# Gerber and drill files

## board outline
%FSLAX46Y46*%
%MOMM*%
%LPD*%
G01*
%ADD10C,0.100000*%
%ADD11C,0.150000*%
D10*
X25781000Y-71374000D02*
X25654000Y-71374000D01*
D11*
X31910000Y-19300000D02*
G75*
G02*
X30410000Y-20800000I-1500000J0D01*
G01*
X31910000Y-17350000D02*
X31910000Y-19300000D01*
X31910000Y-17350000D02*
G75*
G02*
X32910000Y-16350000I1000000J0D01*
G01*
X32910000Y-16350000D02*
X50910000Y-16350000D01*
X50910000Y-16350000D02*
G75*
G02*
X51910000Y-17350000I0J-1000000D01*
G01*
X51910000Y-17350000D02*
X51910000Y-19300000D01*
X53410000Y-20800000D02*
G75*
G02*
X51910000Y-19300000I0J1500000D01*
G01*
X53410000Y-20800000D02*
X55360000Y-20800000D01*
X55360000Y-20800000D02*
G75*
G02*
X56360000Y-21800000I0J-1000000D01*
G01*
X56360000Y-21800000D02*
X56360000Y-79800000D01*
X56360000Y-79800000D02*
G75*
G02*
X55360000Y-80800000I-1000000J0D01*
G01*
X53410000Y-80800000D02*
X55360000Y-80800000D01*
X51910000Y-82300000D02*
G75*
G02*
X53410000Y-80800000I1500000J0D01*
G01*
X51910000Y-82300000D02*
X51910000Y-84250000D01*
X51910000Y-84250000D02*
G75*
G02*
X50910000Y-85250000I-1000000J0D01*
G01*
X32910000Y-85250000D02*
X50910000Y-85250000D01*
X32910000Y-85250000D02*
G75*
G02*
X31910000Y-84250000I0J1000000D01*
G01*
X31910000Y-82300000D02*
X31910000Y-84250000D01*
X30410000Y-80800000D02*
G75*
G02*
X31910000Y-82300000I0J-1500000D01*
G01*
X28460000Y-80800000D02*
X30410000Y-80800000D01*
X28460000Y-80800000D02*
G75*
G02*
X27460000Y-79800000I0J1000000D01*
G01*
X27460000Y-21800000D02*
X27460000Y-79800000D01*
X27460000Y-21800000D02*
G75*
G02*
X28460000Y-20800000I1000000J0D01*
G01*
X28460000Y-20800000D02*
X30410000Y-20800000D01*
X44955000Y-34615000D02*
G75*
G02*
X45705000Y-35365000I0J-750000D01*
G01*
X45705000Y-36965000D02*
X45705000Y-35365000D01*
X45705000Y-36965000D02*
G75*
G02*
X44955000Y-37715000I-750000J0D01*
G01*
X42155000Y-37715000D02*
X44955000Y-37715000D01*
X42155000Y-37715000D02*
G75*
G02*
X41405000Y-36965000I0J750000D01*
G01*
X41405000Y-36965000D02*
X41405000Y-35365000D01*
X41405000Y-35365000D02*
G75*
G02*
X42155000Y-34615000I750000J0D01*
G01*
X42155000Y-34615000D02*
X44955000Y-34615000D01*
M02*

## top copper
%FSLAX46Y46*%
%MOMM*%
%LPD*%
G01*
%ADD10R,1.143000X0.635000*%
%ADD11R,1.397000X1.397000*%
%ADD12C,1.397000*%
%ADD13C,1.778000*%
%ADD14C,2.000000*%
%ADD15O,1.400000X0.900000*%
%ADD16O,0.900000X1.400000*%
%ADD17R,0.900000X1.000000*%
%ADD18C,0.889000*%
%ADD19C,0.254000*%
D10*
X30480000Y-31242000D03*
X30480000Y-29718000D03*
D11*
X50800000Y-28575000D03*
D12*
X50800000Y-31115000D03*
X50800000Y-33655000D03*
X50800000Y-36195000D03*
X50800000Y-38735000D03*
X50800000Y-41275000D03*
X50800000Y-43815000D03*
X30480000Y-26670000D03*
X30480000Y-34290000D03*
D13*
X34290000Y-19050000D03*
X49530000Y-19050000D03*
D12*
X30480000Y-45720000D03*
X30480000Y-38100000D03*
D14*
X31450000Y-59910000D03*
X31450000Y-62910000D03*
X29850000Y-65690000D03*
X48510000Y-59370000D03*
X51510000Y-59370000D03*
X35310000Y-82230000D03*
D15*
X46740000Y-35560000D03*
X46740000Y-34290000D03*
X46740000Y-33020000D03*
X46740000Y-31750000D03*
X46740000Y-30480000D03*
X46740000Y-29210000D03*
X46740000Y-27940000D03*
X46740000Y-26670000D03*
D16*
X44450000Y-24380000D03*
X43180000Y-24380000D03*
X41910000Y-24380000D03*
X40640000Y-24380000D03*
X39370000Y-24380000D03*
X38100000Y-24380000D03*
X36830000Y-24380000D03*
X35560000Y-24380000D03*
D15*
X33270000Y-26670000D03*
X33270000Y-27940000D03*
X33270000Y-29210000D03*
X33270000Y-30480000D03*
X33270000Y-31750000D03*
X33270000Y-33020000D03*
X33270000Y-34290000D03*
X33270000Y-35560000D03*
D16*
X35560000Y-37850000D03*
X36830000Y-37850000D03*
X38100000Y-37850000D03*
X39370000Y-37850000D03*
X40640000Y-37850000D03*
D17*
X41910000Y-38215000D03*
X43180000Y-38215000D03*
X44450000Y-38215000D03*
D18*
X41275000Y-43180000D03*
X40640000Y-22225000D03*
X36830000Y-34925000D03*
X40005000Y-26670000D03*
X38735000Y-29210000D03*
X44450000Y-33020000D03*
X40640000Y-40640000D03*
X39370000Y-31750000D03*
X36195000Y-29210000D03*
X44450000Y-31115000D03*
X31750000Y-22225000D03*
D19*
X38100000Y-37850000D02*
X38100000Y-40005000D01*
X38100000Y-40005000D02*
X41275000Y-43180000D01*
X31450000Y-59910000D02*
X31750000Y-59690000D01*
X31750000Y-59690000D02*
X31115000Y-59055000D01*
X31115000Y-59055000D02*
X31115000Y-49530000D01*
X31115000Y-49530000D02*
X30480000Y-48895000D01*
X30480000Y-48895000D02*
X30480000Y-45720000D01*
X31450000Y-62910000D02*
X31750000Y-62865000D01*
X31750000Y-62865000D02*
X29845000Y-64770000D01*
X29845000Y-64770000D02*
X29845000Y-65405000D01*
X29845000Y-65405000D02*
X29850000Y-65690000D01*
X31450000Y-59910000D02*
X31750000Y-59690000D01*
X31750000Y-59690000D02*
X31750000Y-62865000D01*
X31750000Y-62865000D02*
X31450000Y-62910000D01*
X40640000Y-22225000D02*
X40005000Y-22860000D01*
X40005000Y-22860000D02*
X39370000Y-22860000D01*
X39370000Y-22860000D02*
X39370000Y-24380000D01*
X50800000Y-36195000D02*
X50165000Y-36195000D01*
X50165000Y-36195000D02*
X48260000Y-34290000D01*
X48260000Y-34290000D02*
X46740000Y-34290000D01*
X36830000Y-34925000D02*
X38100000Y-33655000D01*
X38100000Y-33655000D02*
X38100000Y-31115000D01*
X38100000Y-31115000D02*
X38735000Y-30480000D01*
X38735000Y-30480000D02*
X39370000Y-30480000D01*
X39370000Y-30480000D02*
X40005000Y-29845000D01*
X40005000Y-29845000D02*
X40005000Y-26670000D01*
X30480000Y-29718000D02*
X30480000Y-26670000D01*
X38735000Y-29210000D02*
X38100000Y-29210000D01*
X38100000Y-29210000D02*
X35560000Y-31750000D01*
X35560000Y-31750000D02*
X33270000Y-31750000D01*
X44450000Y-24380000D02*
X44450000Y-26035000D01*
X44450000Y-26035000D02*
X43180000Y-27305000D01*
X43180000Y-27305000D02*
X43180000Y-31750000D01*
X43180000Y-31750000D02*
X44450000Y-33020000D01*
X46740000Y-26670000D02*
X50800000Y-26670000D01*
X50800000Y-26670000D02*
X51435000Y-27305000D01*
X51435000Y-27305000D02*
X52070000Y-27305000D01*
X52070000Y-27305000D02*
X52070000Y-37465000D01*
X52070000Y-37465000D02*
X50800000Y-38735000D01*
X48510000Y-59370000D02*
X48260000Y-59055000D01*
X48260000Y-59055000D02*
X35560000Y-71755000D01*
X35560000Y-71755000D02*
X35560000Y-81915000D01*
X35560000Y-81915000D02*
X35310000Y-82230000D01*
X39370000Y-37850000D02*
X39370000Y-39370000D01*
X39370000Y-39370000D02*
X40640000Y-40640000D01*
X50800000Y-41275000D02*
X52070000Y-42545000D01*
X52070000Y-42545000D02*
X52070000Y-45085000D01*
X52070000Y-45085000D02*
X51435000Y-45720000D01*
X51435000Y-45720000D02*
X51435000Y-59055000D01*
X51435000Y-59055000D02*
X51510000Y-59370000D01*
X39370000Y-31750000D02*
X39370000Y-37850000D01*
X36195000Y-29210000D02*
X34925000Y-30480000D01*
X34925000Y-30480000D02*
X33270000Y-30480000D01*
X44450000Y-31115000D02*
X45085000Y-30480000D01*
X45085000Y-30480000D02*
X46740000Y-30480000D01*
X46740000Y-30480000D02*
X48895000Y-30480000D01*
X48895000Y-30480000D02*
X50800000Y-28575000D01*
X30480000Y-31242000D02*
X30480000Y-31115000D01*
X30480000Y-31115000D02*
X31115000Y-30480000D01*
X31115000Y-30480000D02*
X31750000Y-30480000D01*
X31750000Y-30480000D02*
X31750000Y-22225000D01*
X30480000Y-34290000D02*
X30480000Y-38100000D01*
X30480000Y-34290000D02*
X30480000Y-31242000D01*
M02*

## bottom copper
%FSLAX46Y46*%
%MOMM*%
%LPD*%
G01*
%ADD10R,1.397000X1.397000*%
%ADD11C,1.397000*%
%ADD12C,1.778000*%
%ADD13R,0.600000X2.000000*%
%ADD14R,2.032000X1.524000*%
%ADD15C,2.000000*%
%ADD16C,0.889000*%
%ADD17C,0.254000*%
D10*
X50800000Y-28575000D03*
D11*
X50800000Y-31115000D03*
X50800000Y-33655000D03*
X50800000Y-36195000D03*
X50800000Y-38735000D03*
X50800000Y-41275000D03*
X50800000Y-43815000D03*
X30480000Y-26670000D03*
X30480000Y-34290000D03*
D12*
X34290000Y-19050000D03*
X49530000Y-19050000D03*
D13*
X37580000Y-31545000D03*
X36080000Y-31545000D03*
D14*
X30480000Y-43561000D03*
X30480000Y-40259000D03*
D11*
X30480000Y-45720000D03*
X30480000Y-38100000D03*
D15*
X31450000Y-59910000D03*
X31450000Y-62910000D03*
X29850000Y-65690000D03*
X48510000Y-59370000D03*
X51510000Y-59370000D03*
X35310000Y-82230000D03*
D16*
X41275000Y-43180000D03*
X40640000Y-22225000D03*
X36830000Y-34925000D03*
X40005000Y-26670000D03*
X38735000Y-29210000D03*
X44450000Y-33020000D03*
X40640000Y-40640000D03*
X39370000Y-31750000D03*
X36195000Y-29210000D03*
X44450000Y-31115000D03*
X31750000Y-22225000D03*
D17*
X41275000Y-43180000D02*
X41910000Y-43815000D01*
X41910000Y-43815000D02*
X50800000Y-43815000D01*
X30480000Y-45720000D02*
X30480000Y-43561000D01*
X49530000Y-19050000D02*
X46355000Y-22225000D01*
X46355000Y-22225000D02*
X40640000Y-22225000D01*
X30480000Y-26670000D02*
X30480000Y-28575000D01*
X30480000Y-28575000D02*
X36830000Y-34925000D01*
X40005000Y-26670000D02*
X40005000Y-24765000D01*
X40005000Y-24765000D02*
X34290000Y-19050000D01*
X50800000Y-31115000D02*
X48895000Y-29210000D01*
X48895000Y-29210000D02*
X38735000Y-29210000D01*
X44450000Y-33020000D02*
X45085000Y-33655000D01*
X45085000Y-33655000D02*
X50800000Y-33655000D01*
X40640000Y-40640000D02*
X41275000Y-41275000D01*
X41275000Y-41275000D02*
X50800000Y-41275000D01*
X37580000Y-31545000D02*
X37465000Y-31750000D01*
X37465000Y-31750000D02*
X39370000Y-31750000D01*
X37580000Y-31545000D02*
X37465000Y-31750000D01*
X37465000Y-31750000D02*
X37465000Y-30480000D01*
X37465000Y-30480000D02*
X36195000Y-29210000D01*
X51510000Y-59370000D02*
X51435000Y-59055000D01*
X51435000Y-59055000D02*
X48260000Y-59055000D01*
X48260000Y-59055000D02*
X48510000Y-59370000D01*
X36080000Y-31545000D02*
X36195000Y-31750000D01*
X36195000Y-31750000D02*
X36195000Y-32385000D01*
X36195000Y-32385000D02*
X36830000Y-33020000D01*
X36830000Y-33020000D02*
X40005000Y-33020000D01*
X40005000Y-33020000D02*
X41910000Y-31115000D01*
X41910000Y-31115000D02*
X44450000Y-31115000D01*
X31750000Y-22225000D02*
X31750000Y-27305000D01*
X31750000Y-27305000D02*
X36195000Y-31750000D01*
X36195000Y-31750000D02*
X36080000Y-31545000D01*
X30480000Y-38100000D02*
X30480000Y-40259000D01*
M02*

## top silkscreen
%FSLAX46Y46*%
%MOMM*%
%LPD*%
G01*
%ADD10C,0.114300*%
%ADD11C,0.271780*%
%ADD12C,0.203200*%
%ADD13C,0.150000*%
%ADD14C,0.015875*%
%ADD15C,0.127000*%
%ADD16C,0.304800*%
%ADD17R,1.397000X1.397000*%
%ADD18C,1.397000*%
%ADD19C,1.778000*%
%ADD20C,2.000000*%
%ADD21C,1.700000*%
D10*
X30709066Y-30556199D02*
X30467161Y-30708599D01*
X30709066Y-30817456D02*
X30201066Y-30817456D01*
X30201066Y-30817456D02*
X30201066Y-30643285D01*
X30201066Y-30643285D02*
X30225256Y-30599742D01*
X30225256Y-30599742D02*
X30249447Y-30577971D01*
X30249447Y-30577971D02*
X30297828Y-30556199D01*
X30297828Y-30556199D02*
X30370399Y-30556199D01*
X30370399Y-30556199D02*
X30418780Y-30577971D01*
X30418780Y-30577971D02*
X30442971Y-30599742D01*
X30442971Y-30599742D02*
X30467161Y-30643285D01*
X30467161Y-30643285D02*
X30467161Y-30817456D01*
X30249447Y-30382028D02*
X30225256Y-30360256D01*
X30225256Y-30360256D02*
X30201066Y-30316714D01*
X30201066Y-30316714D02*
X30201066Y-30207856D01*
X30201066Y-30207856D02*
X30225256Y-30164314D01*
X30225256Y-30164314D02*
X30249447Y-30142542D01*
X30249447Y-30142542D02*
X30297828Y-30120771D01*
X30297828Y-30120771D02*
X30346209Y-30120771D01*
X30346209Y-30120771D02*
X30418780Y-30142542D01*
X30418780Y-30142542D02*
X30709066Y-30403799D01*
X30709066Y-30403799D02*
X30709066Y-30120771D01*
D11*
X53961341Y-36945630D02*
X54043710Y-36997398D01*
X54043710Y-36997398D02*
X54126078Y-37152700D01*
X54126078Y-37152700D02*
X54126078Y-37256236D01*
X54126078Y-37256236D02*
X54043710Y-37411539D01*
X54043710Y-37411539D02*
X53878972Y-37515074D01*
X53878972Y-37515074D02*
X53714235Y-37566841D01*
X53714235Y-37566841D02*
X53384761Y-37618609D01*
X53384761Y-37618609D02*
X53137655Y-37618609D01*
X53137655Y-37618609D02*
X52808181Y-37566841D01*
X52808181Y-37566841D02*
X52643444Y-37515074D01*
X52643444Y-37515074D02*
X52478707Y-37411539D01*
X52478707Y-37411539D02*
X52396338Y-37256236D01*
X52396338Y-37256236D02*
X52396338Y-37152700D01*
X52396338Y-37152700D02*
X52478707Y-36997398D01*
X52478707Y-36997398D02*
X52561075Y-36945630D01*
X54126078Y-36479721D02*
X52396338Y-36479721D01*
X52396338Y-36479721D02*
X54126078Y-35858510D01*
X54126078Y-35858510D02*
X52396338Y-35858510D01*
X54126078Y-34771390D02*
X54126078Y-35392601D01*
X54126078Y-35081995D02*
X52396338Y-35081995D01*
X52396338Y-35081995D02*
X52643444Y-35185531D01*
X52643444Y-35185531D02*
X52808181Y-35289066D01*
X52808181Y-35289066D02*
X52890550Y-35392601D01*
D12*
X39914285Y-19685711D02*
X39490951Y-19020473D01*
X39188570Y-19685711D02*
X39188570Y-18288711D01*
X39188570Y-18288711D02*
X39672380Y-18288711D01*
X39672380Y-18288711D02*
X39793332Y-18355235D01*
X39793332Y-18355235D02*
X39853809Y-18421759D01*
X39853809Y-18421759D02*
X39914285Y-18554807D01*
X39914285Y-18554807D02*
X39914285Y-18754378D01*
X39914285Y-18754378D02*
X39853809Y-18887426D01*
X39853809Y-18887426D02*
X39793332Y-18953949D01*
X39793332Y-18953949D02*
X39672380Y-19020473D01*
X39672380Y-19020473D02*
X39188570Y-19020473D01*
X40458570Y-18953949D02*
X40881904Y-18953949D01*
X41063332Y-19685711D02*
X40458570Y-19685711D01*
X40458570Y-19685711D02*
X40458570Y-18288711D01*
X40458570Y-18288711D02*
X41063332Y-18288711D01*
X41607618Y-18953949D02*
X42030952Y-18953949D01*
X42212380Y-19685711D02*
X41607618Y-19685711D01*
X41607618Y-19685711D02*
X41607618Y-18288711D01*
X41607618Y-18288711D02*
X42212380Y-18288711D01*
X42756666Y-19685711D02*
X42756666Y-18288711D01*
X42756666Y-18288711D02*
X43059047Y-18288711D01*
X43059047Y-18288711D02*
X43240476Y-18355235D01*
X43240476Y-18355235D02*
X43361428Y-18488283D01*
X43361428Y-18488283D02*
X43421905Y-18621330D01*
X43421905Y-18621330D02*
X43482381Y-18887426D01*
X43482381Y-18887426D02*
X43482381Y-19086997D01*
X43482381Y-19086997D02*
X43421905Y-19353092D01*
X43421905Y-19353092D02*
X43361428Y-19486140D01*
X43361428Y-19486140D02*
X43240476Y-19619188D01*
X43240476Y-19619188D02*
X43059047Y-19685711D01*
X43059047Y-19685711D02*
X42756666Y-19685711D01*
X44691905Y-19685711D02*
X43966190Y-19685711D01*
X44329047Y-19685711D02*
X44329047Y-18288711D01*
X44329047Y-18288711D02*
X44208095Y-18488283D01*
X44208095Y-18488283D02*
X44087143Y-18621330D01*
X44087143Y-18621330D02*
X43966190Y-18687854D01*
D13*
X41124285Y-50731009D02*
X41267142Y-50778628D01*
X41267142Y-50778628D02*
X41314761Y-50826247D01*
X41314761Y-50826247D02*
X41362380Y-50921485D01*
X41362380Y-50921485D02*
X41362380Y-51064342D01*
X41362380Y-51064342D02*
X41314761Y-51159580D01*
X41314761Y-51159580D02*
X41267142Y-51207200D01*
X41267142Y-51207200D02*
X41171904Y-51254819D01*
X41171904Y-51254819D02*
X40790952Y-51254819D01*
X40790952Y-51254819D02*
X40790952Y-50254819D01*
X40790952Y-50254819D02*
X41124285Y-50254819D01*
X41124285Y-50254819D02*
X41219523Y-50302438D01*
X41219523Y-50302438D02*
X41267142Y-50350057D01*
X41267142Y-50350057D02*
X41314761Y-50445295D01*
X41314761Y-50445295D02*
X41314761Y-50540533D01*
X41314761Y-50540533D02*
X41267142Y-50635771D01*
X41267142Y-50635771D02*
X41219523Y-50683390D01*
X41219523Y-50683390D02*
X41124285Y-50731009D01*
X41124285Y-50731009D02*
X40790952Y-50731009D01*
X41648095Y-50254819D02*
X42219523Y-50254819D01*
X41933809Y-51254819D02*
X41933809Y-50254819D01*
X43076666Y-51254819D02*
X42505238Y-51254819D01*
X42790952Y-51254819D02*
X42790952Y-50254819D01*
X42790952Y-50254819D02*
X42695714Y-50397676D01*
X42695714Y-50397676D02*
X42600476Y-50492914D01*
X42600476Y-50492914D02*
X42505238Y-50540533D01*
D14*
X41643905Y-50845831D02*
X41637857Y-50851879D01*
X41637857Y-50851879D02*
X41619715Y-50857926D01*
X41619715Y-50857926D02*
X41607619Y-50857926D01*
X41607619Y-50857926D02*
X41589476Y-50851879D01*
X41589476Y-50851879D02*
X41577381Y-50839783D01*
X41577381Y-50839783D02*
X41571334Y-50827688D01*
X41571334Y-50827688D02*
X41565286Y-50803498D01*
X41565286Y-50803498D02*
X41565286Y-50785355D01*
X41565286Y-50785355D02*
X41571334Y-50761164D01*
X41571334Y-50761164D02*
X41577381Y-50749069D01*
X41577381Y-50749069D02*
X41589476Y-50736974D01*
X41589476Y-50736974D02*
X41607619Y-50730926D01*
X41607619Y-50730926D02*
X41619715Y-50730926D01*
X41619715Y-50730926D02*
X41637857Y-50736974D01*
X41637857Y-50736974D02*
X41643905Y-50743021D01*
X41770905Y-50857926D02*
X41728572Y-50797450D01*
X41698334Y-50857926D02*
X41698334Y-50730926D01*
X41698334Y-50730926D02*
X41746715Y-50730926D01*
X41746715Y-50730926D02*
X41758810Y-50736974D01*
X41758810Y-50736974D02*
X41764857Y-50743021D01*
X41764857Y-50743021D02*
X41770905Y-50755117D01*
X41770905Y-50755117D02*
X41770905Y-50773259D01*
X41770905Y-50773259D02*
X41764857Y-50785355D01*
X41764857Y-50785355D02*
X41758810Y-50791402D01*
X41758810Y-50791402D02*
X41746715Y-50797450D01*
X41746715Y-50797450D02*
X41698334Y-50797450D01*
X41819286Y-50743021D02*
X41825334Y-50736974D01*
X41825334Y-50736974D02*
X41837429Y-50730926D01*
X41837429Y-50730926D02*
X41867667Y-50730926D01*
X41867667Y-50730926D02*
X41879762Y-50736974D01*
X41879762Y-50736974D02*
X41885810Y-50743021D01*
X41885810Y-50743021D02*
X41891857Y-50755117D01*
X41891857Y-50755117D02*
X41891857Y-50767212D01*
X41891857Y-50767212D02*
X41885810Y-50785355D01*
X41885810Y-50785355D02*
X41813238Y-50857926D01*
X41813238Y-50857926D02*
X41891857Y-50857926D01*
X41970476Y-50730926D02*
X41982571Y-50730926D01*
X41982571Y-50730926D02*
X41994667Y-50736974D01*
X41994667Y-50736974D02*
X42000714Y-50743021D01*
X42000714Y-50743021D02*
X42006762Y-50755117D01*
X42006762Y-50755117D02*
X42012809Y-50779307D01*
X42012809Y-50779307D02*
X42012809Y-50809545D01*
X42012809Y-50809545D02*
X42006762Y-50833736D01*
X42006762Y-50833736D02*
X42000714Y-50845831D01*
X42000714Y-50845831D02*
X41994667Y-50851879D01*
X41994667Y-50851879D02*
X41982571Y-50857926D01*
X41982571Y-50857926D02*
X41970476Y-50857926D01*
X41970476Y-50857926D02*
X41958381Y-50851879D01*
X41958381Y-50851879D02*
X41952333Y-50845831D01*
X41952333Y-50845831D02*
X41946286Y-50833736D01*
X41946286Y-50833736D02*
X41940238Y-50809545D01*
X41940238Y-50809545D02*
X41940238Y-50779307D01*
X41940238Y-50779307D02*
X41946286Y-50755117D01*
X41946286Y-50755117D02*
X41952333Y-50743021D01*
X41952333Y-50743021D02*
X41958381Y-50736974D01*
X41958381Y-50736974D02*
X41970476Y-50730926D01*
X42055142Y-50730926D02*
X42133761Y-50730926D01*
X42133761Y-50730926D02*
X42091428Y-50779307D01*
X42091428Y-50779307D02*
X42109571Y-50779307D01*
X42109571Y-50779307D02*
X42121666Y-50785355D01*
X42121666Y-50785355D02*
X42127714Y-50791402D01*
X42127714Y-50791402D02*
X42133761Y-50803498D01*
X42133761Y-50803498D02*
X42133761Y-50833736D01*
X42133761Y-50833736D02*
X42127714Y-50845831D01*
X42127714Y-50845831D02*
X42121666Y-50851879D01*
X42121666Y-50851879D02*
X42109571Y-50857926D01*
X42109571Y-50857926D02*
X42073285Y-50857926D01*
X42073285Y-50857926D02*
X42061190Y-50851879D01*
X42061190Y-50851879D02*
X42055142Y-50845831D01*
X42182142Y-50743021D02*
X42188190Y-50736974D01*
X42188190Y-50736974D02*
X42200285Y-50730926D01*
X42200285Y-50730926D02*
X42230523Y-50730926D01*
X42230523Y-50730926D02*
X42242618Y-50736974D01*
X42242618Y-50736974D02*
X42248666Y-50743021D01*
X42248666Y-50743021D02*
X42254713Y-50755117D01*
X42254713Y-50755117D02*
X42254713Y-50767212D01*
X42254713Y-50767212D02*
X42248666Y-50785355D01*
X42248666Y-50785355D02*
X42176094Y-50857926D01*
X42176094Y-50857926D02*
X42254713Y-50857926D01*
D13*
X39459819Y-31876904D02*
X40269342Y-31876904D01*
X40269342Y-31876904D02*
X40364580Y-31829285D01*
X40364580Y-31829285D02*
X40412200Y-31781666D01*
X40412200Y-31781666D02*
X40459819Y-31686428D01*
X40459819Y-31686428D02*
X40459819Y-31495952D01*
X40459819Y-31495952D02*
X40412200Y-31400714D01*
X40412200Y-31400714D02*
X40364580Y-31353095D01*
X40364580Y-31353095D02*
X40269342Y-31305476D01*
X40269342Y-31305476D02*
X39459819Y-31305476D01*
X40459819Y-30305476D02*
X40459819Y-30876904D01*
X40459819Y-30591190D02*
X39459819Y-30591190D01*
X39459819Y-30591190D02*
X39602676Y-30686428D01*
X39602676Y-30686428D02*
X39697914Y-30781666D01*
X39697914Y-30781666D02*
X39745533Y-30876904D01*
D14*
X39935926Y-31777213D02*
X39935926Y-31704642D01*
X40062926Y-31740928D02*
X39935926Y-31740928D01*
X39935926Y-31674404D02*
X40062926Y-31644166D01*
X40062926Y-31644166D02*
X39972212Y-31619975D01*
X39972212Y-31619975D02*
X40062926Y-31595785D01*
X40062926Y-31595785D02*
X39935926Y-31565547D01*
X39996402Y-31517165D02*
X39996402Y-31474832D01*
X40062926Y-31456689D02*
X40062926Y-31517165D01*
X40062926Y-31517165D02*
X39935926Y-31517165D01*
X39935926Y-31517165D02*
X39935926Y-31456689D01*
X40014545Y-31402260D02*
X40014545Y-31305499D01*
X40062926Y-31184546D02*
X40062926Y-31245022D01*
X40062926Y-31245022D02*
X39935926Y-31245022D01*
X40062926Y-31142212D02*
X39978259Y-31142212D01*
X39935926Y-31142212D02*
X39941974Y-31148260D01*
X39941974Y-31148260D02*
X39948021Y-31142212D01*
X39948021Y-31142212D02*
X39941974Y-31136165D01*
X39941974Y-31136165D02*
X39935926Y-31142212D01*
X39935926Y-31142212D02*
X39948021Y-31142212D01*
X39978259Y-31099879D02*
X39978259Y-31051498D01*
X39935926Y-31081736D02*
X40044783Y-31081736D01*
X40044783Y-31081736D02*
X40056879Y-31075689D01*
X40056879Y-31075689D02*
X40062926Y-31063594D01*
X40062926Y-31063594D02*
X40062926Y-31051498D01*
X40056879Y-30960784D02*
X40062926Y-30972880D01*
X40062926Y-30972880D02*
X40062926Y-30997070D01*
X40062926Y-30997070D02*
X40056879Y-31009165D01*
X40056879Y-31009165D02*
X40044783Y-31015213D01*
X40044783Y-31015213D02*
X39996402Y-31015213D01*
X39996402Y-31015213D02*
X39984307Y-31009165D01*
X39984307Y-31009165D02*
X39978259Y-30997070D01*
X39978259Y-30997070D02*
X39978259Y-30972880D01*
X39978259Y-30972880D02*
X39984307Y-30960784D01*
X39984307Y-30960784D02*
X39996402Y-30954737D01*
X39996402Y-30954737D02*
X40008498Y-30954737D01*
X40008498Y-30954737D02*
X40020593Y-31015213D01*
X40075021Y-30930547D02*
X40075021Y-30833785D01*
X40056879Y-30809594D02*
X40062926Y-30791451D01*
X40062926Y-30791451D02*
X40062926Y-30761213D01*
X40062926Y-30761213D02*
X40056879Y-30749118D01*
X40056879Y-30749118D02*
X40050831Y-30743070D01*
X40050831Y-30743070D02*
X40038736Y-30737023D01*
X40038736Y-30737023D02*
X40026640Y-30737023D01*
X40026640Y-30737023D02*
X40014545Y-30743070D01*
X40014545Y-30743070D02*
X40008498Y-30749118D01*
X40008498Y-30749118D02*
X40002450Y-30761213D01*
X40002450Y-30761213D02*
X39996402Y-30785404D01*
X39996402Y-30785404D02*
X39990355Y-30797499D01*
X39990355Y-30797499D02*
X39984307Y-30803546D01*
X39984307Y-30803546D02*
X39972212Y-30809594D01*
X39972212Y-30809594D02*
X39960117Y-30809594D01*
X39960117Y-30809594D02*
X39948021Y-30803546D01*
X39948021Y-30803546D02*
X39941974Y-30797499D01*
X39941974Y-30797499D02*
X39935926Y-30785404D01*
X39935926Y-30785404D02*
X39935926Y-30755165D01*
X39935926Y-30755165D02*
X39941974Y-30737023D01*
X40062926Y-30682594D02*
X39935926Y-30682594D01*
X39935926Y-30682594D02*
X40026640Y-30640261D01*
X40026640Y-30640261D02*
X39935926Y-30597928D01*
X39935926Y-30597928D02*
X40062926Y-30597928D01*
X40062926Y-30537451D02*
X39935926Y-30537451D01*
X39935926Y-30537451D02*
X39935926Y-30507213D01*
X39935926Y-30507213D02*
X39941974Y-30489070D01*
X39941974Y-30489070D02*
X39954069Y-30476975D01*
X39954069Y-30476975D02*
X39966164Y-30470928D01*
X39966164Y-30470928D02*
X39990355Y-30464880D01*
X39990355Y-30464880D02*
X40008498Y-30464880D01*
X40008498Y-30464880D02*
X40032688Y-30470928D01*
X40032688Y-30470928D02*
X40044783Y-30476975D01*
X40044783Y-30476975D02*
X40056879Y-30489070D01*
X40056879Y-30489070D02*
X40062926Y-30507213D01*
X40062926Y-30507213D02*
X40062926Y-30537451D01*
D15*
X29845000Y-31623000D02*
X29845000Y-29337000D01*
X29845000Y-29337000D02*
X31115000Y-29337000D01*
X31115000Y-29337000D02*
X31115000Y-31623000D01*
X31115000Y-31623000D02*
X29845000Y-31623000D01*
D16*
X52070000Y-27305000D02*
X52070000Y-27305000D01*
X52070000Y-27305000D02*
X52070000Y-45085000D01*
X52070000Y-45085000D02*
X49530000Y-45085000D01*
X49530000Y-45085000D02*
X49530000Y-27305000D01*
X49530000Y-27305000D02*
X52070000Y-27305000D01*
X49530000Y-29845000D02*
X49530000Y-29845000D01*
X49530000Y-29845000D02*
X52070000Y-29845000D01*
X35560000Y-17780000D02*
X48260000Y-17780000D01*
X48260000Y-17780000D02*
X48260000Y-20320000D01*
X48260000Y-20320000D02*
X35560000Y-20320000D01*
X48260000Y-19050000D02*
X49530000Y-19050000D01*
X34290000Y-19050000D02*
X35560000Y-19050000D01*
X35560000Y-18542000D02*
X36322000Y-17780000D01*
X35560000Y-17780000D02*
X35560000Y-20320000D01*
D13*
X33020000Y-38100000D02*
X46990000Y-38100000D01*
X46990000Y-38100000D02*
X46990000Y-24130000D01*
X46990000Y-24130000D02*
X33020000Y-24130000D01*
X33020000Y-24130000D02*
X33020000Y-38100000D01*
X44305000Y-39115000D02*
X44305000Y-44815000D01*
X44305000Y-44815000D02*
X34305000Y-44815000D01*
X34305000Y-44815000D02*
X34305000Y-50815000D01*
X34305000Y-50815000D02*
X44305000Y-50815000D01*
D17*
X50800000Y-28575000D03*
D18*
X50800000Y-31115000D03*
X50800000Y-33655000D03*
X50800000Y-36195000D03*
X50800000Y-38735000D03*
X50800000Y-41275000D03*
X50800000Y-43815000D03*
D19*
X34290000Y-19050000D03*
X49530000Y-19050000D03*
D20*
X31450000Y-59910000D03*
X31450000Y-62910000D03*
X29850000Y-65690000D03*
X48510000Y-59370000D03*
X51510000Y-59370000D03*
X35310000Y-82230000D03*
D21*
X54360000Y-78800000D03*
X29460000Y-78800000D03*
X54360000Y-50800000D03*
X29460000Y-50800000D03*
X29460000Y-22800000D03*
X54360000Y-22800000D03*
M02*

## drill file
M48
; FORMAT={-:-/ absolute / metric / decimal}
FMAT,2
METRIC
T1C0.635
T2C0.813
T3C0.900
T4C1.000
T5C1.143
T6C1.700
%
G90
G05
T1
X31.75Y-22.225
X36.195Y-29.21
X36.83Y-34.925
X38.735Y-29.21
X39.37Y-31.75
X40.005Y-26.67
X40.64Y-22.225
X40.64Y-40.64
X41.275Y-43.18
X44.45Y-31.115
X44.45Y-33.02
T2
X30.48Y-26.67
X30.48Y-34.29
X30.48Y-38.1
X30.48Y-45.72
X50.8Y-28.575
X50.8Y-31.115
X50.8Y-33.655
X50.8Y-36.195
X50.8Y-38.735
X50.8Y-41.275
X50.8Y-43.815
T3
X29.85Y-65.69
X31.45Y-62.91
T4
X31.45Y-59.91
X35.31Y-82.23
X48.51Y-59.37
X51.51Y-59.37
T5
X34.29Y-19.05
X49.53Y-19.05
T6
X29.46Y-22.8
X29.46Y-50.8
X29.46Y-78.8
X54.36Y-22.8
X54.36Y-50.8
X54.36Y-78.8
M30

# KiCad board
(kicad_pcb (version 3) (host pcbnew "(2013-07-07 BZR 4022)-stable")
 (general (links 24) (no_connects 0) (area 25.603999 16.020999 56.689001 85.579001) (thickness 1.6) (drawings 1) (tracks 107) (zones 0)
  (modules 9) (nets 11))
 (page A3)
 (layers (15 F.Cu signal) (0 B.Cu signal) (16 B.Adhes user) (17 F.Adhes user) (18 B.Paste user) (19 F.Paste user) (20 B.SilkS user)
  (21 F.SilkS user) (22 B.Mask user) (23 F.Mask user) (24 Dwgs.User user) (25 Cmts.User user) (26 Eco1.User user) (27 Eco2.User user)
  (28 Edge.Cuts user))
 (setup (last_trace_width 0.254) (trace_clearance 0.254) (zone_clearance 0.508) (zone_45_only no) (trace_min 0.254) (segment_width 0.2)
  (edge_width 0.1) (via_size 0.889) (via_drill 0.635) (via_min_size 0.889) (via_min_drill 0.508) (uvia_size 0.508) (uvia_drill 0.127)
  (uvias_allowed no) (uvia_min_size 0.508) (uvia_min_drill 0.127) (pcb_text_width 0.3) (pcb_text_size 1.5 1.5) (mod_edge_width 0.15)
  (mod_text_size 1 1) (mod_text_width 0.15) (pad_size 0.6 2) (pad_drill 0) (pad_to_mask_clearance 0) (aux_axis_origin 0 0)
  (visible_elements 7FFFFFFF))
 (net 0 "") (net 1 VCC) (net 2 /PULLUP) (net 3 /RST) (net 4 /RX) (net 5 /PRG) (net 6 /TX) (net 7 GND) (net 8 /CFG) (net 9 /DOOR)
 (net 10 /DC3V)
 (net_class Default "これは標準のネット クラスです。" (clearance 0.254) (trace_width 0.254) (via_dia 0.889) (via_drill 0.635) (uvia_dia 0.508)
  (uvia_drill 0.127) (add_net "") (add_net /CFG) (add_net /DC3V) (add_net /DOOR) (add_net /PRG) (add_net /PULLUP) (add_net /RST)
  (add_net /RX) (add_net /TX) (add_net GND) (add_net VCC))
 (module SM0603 (layer F.Cu) (at 30.48 30.48 90)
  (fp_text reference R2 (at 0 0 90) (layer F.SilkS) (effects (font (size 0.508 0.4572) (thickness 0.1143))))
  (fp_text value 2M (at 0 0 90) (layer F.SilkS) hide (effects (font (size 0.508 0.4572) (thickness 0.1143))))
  (fp_line (start -1.143 -0.635) (end 1.143 -0.635) (layer F.SilkS) (width 0.127))
  (fp_line (start 1.143 -0.635) (end 1.143 0.635) (layer F.SilkS) (width 0.127))
  (fp_line (start 1.143 0.635) (end -1.143 0.635) (layer F.SilkS) (width 0.127))
  (fp_line (start -1.143 0.635) (end -1.143 -0.635) (layer F.SilkS) (width 0.127))
  (pad 1 smd rect (at -0.762 0 90) (size 0.635 1.143) (layers F.Cu F.Paste F.Mask) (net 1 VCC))
  (pad 2 smd rect (at 0.762 0 90) (size 0.635 1.143) (layers F.Cu F.Paste F.Mask) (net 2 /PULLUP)))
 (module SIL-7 (layer F.Cu) (at 50.8 36.195 270)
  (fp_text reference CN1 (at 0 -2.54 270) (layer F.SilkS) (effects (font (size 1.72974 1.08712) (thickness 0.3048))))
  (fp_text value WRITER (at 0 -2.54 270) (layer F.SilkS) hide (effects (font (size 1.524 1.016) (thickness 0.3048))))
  (fp_line (start -8.89 -1.27) (end -8.89 -1.27) (layer F.SilkS) (width 0.3048))
  (fp_line (start -8.89 -1.27) (end 8.89 -1.27) (layer F.SilkS) (width 0.3048))
  (fp_line (start 8.89 -1.27) (end 8.89 1.27) (layer F.SilkS) (width 0.3048))
  (fp_line (start 8.89 1.27) (end -8.89 1.27) (layer F.SilkS) (width 0.3048))
  (fp_line (start -8.89 1.27) (end -8.89 -1.27) (layer F.SilkS) (width 0.3048))
  (fp_line (start -6.35 1.27) (end -6.35 1.27) (layer F.SilkS) (width 0.3048))
  (fp_line (start -6.35 1.27) (end -6.35 -1.27) (layer F.SilkS) (width 0.3048))
  (pad 1 thru_hole rect (at -7.62 0 270) (size 1.397 1.397) (drill 0.8128) (layers *.Cu *.Mask F.SilkS) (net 1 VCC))
  (pad 2 thru_hole circle (at -5.08 0 270) (size 1.397 1.397) (drill 0.8128) (layers *.Cu *.SilkS *.Mask) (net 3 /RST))
  (pad 3 thru_hole circle (at -2.54 0 270) (size 1.397 1.397) (drill 0.8128) (layers *.Cu *.SilkS *.Mask) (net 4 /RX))
  (pad 4 thru_hole circle (at 0 0 270) (size 1.397 1.397) (drill 0.8128) (layers *.Cu *.SilkS *.Mask) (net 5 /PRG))
  (pad 5 thru_hole circle (at 2.54 0 270) (size 1.397 1.397) (drill 0.8128) (layers *.Cu *.SilkS *.Mask) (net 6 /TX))
  (pad 6 thru_hole circle (at 5.08 0 270) (size 1.397 1.397) (drill 0.8128) (layers *.Cu *.SilkS *.Mask) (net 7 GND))
  (pad 7 thru_hole circle (at 7.62 0 270) (size 1.397 1.397) (drill 0.8128) (layers *.Cu *.SilkS *.Mask) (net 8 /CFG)))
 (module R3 (layer B.Cu) (at 30.48 30.48 270) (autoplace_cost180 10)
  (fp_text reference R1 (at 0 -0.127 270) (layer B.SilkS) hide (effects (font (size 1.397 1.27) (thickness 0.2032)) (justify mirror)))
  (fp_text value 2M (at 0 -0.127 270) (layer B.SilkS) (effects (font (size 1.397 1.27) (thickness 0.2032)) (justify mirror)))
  (pad 1 thru_hole circle (at -3.81 0 270) (size 1.397 1.397) (drill 0.8128) (layers *.Cu *.Mask B.SilkS) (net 2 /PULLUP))
  (pad 2 thru_hole circle (at 3.81 0 270) (size 1.397 1.397) (drill 0.8128) (layers *.Cu *.Mask B.SilkS) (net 1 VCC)))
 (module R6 (layer F.Cu) (at 41.91 19.05) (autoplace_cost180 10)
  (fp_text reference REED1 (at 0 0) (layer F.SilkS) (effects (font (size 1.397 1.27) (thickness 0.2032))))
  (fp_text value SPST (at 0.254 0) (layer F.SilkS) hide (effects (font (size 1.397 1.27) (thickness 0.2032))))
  (fp_line (start -6.35 -1.27) (end 6.35 -1.27) (layer F.SilkS) (width 0.3048))
  (fp_line (start 6.35 -1.27) (end 6.35 1.27) (layer F.SilkS) (width 0.3048))
  (fp_line (start 6.35 1.27) (end -6.35 1.27) (layer F.SilkS) (width 0.3048))
  (fp_line (start 6.35 0) (end 7.62 0) (layer F.SilkS) (width 0.3048))
  (fp_line (start -7.62 0) (end -6.35 0) (layer F.SilkS) (width 0.3048))
  (fp_line (start -6.35 -0.508) (end -5.588 -1.27) (layer F.SilkS) (width 0.3048))
  (fp_line (start -6.35 -1.27) (end -6.35 1.27) (layer F.SilkS) (width 0.3048))
  (pad 1 thru_hole circle (at -7.62 0) (size 1.778 1.778) (drill 1.143) (layers *.Cu *.Mask F.SilkS) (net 2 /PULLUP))
  (pad 2 thru_hole circle (at 7.62 0) (size 1.778 1.778) (drill 1.143) (layers *.Cu *.Mask F.SilkS) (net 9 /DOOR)))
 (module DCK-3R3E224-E (layer B.Cu) (at 36.83 36.195)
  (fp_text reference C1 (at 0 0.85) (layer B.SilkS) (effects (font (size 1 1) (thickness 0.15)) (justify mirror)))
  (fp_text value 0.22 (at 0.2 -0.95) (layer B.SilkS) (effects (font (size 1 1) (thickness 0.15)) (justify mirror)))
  (pad 1 smd rect (at 0.75 -4.65) (size 0.6 2) (layers B.Cu B.Paste B.Mask) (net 7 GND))
  (pad 2 smd rect (at -0.75 -4.65) (size 0.6 2) (layers B.Cu B.Paste B.Mask) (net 1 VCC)))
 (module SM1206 (layer B.Cu) (at 30.48 41.91 90)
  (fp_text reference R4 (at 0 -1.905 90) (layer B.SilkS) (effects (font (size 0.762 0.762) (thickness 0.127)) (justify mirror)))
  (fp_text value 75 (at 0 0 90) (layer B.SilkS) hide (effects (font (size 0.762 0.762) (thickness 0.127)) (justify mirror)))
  (pad 1 smd rect (at -1.651 0 90) (size 1.524 2.032) (layers B.Cu B.Paste B.Mask) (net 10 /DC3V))
  (pad 2 smd rect (at 1.651 0 90) (size 1.524 2.032) (layers B.Cu B.Paste B.Mask) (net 1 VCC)))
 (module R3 (layer B.Cu) (at 30.48 41.91 90) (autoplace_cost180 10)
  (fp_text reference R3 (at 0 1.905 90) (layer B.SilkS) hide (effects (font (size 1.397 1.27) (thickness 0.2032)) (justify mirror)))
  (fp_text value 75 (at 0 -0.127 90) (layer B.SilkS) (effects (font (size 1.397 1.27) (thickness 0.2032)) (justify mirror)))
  (pad 1 thru_hole circle (at -3.81 0 90) (size 1.397 1.397) (drill 0.8128) (layers *.Cu *.Mask B.SilkS) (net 10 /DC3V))
  (pad 2 thru_hole circle (at 3.81 0 90) (size 1.397 1.397) (drill 0.8128) (layers *.Cu *.Mask B.SilkS) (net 1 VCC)))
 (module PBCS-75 (layer F.Cu) (at 41.91 50.8)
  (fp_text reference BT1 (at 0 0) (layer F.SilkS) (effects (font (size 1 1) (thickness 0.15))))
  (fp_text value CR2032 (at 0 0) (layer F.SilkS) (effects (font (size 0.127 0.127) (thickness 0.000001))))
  (fp_arc (start -11.5 -31.5) (end -10 -31.5) (angle 90) (layer Edge.Cuts) (width 0.15))
  (fp_line (start -10 -33.45) (end -10 -31.5) (layer Edge.Cuts) (width 0.15))
  (fp_arc (start -9 -33.45) (end -10 -33.45) (angle 90) (layer Edge.Cuts) (width 0.15))
  (fp_line (start -9 -34.45) (end 9 -34.45) (layer Edge.Cuts) (width 0.15))
  (fp_arc (start 9 -33.45) (end 9 -34.45) (angle 90) (layer Edge.Cuts) (width 0.15))
  (fp_line (start 10 -33.45) (end 10 -31.5) (layer Edge.Cuts) (width 0.15))
  (fp_arc (start 11.5 -31.5) (end 11.5 -30) (angle 90) (layer Edge.Cuts) (width 0.15))
  (fp_line (start 11.5 -30) (end 13.45 -30) (layer Edge.Cuts) (width 0.15))
  (fp_arc (start 13.45 -29) (end 13.45 -30) (angle 90) (layer Edge.Cuts) (width 0.15))
  (fp_line (start 14.45 -29) (end 14.45 29) (layer Edge.Cuts) (width 0.15))
  (fp_arc (start 13.45 29) (end 14.45 29) (angle 90) (layer Edge.Cuts) (width 0.15))
  (fp_line (start 11.5 30) (end 13.45 30) (layer Edge.Cuts) (width 0.15))
  (fp_arc (start 11.5 31.5) (end 10 31.5) (angle 90) (layer Edge.Cuts) (width 0.15))
  (fp_line (start 10 31.5) (end 10 33.45) (layer Edge.Cuts) (width 0.15))
  (fp_arc (start 9 33.45) (end 10 33.45) (angle 90) (layer Edge.Cuts) (width 0.15))
  (fp_line (start -9 34.45) (end 9 34.45) (layer Edge.Cuts) (width 0.15))
  (fp_arc (start -9 33.45) (end -9 34.45) (angle 90) (layer Edge.Cuts) (width 0.15))
  (fp_line (start -10 31.5) (end -10 33.45) (layer Edge.Cuts) (width 0.15))
  (fp_arc (start -11.5 31.5) (end -11.5 30) (angle 90) (layer Edge.Cuts) (width 0.15))
  (fp_line (start -13.45 30) (end -11.5 30) (layer Edge.Cuts) (width 0.15))
  (fp_arc (start -13.45 29) (end -13.45 30) (angle 90) (layer Edge.Cuts) (width 0.15))
  (fp_line (start -14.45 -29) (end -14.45 29) (layer Edge.Cuts) (width 0.15))
  (fp_arc (start -13.45 -29) (end -14.45 -29) (angle 90) (layer Edge.Cuts) (width 0.15))
  (fp_line (start -13.45 -30) (end -11.5 -30) (layer Edge.Cuts) (width 0.15))
  (pad 1 thru_hole circle (at -10.46 9.11) (size 2 2) (drill 1) (layers *.Cu *.Mask F.SilkS) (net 10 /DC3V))
  (pad 1 thru_hole circle (at -10.46 12.11) (size 2 2) (drill 0.9) (layers *.Cu *.Mask F.SilkS) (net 10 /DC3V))
  (pad 1 thru_hole circle (at -12.06 14.89) (size 2 2) (drill 0.9) (layers *.Cu *.Mask F.SilkS) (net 10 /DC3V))
  (pad 2 thru_hole circle (at 6.6 8.57) (size 2 2) (drill 1) (layers *.Cu *.Mask F.SilkS) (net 7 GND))
  (pad 2 thru_hole circle (at 9.6 8.57) (size 2 2) (drill 1) (layers *.Cu *.Mask F.SilkS) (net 7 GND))
  (pad 2 thru_hole circle (at -6.6 31.43) (size 2 2) (drill 1) (layers *.Cu *.Mask F.SilkS) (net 7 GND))
  (pad "" np_thru_hole circle (at 12.45 28) (size 1.7 1.7) (drill 1.7) (layers *.Cu *.Mask F.SilkS))
  (pad "" np_thru_hole circle (at -12.45 28) (size 1.7 1.7) (drill 1.7) (layers *.Cu *.Mask F.SilkS))
  (pad "" np_thru_hole circle (at 12.45 0) (size 1.7 1.7) (drill 1.7) (layers *.Cu *.Mask F.SilkS))
  (pad "" np_thru_hole circle (at -12.45 0) (size 1.7 1.7) (drill 1.7) (layers *.Cu *.Mask F.SilkS))
  (pad "" np_thru_hole circle (at -12.45 -28) (size 1.7 1.7) (drill 1.7) (layers *.Cu *.Mask F.SilkS))
  (pad "" np_thru_hole circle (at 12.45 -28) (size 1.7 1.7) (drill 1.7) (layers *.Cu *.Mask F.SilkS)))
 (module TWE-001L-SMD (layer F.Cu) (at 40.005 31.115 90)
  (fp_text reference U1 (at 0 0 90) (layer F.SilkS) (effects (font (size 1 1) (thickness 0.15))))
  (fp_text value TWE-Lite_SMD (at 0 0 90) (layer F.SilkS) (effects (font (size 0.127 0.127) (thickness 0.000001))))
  (fp_arc (start -4.25 4.95) (end -3.5 4.95) (angle 90) (layer Edge.Cuts) (width 0.15))
  (fp_line (start -5.85 5.7) (end -4.25 5.7) (layer Edge.Cuts) (width 0.15))
  (fp_arc (start -5.85 4.95) (end -5.85 5.7) (angle 90) (layer Edge.Cuts) (width 0.15))
  (fp_line (start -6.6 2.15) (end -6.6 4.95) (layer Edge.Cuts) (width 0.15))
  (fp_arc (start -5.85 2.15) (end -6.6 2.15) (angle 90) (layer Edge.Cuts) (width 0.15))
  (fp_line (start -5.85 1.4) (end -4.25 1.4) (layer Edge.Cuts) (width 0.15))
  (fp_arc (start -4.25 2.15) (end -4.25 1.4) (angle 90) (layer Edge.Cuts) (width 0.15))
  (fp_line (start -3.5 2.15) (end -3.5 4.95) (layer Edge.Cuts) (width 0.15))
  (fp_line (start -6.985 -6.985) (end -6.985 6.985) (layer F.SilkS) (width 0.15))
  (fp_line (start -6.985 6.985) (end 6.985 6.985) (layer F.SilkS) (width 0.15))
  (fp_line (start 6.985 6.985) (end 6.985 -6.985) (layer F.SilkS) (width 0.15))
  (fp_line (start 6.985 -6.985) (end -6.985 -6.985) (layer F.SilkS) (width 0.15))
  (fp_line (start -8 4.3) (end -13.7 4.3) (layer F.SilkS) (width 0.15))
  (fp_line (start -13.7 4.3) (end -13.7 -5.7) (layer F.SilkS) (width 0.15))
  (fp_line (start -13.7 -5.7) (end -19.7 -5.7) (layer F.SilkS) (width 0.15))
  (fp_line (start -19.7 -5.7) (end -19.7 4.3) (layer F.SilkS) (width 0.15))
  (pad 1 smd oval (at -4.445 6.735 90) (size 0.9 1.4) (layers F.Cu F.Paste F.Mask))
  (pad 2 smd oval (at -3.175 6.735 90) (size 0.9 1.4) (layers F.Cu F.Paste F.Mask) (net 5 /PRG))
  (pad 3 smd oval (at -1.905 6.735 90) (size 0.9 1.4) (layers F.Cu F.Paste F.Mask))
  (pad 4 smd oval (at -0.635 6.735 90) (size 0.9 1.4) (layers F.Cu F.Paste F.Mask))
  (pad 5 smd oval (at 0.635 6.735 90) (size 0.9 1.4) (layers F.Cu F.Paste F.Mask) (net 1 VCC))
  (pad 6 smd oval (at 1.905 6.735 90) (size 0.9 1.4) (layers F.Cu F.Paste F.Mask))
  (pad 7 smd oval (at 3.175 6.735 90) (size 0.9 1.4) (layers F.Cu F.Paste F.Mask))
  (pad 8 smd oval (at 4.445 6.735 90) (size 0.9 1.4) (layers F.Cu F.Paste F.Mask) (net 6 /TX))
  (pad 9 smd oval (at 6.735 4.445 180) (size 0.9 1.4) (layers F.Cu F.Paste F.Mask) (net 4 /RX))
  (pad 10 smd oval (at 6.735 3.175 180) (size 0.9 1.4) (layers F.Cu F.Paste F.Mask))
  (pad 11 smd oval (at 6.735 1.905 180) (size 0.9 1.4) (layers F.Cu F.Paste F.Mask))
  (pad 12 smd oval (at 6.735 0.635 180) (size 0.9 1.4) (layers F.Cu F.Paste F.Mask))
  (pad 13 smd oval (at 6.735 -0.635 180) (size 0.9 1.4) (layers F.Cu F.Paste F.Mask) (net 9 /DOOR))
  (pad 14 smd oval (at 6.735 -1.905 180) (size 0.9 1.4) (layers F.Cu F.Paste F.Mask))
  (pad 15 smd oval (at 6.735 -3.175 180) (size 0.9 1.4) (layers F.Cu F.Paste F.Mask))
  (pad 16 smd oval (at 6.735 -4.445 180) (size 0.9 1.4) (layers F.Cu F.Paste F.Mask))
  (pad 17 smd oval (at 4.445 -6.735 90) (size 0.9 1.4) (layers F.Cu F.Paste F.Mask))
  (pad 18 smd oval (at 3.175 -6.735 90) (size 0.9 1.4) (layers F.Cu F.Paste F.Mask))
  (pad 19 smd oval (at 1.905 -6.735 90) (size 0.9 1.4) (layers F.Cu F.Paste F.Mask))
  (pad 20 smd oval (at 0.635 -6.735 90) (size 0.9 1.4) (layers F.Cu F.Paste F.Mask) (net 7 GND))
  (pad 21 smd oval (at -0.635 -6.735 90) (size 0.9 1.4) (layers F.Cu F.Paste F.Mask) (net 3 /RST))
  (pad 22 smd oval (at -1.905 -6.735 90) (size 0.9 1.4) (layers F.Cu F.Paste F.Mask))
  (pad 23 smd oval (at -3.175 -6.735 90) (size 0.9 1.4) (layers F.Cu F.Paste F.Mask))
  (pad 24 smd oval (at -4.445 -6.735 90) (size 0.9 1.4) (layers F.Cu F.Paste F.Mask))
  (pad 25 smd oval (at -6.735 -4.445 180) (size 0.9 1.4) (layers F.Cu F.Paste F.Mask))
  (pad 26 smd oval (at -6.735 -3.175 180) (size 0.9 1.4) (layers F.Cu F.Paste F.Mask))
  (pad 27 smd oval (at -6.735 -1.905 180) (size 0.9 1.4) (layers F.Cu F.Paste F.Mask) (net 8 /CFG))
  (pad 28 smd oval (at -6.735 -0.635 180) (size 0.9 1.4) (layers F.Cu F.Paste F.Mask) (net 7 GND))
  (pad 29 smd oval (at -6.735 0.635 180) (size 0.9 1.4) (layers F.Cu F.Paste F.Mask))
  (pad 30 smd rect (at -7.1 1.905 180) (size 0.9 1) (layers F.Cu F.Paste F.Mask))
  (pad 31 smd rect (at -7.1 3.175 180) (size 0.9 1) (layers F.Cu F.Paste F.Mask))
  (pad 32 smd rect (at -7.1 4.445 180) (size 0.9 1) (layers F.Cu F.Paste F.Mask)))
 (gr_line (start 25.781 71.374) (end 25.654 71.374) (angle 90) (layer Edge.Cuts) (width 0.1))
 (segment (start 38.1 37.85) (end 38.1 40.005) (width 0.254) (layer F.Cu) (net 8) (status 80000))
 (segment (start 38.1 40.005) (end 41.275 43.18) (width 0.254) (layer F.Cu) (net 8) (status 80000))
 (via (at 41.275 43.18) (size 0.889) (layers F.Cu B.Cu) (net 8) (status 80000))
 (segment (start 41.275 43.18) (end 41.91 43.815) (width 0.254) (layer B.Cu) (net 8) (status 80000))
 (segment (start 41.91 43.815) (end 50.8 43.815) (width 0.254) (layer B.Cu) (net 8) (status 80000))
 (segment (start 31.45 59.91) (end 31.75 59.69) (width 0.254) (layer F.Cu) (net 10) (status 80000))
 (segment (start 31.75 59.69) (end 31.115 59.055) (width 0.254) (layer F.Cu) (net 10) (status 80000))
 (segment (start 31.115 59.055) (end 31.115 49.53) (width 0.254) (layer F.Cu) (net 10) (status 80000))
 (segment (start 31.115 49.53) (end 30.48 48.895) (width 0.254) (layer F.Cu) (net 10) (status 80000))
 (segment (start 30.48 48.895) (end 30.48 45.72) (width 0.254) (layer F.Cu) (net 10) (status 80000))
 (segment (start 31.45 62.91) (end 31.75 62.865) (width 0.254) (layer F.Cu) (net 10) (status 80000))
 (segment (start 31.75 62.865) (end 29.845 64.77) (width 0.254) (layer F.Cu) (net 10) (status 80000))
 (segment (start 29.845 64.77) (end 29.845 65.405) (width 0.254) (layer F.Cu) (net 10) (status 80000))
 (segment (start 29.845 65.405) (end 29.85 65.69) (width 0.254) (layer F.Cu) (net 10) (status 80000))
 (segment (start 31.45 59.91) (end 31.75 59.69) (width 0.254) (layer F.Cu) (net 10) (status 80000))
 (segment (start 31.75 59.69) (end 31.75 62.865) (width 0.254) (layer F.Cu) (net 10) (status 80000))
 (segment (start 31.75 62.865) (end 31.45 62.91) (width 0.254) (layer F.Cu) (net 10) (status 80000))
 (segment (start 30.48 45.72) (end 30.48 43.561) (width 0.254) (layer B.Cu) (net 10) (status 80000))
 (segment (start 49.53 19.05) (end 46.355 22.225) (width 0.254) (layer B.Cu) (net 9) (status 80000))
 (segment (start 46.355 22.225) (end 40.64 22.225) (width 0.254) (layer B.Cu) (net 9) (status 80000))
 (via (at 40.64 22.225) (size 0.889) (layers F.Cu B.Cu) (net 9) (status 80000))
 (segment (start 40.64 22.225) (end 40.005 22.86) (width 0.254) (layer F.Cu) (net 9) (status 80000))
 (segment (start 40.005 22.86) (end 39.37 22.86) (width 0.254) (layer F.Cu) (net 9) (status 80000))
 (segment (start 39.37 22.86) (end 39.37 24.38) (width 0.254) (layer F.Cu) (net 9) (status 80000))
 (segment (start 50.8 36.195) (end 50.165 36.195) (width 0.254) (layer F.Cu) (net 5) (status 80000))
 (segment (start 50.165 36.195) (end 48.26 34.29) (width 0.254) (layer F.Cu) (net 5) (status 80000))
 (segment (start 48.26 34.29) (end 46.74 34.29) (width 0.254) (layer F.Cu) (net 5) (status 80000))
 (segment (start 30.48 26.67) (end 30.48 28.575) (width 0.254) (layer B.Cu) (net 2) (status 80000))
 (segment (start 30.48 28.575) (end 36.83 34.925) (width 0.254) (layer B.Cu) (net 2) (status 80000))
 (via (at 36.83 34.925) (size 0.889) (layers F.Cu B.Cu) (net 2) (status 80000))
 (segment (start 36.83 34.925) (end 38.1 33.655) (width 0.254) (layer F.Cu) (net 2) (status 80000))
 (segment (start 38.1 33.655) (end 38.1 31.115) (width 0.254) (layer F.Cu) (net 2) (status 80000))
 (segment (start 38.1 31.115) (end 38.735 30.48) (width 0.254) (layer F.Cu) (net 2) (status 80000))
 (segment (start 38.735 30.48) (end 39.37 30.48) (width 0.254) (layer F.Cu) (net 2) (status 80000))
 (segment (start 39.37 30.48) (end 40.005 29.845) (width 0.254) (layer F.Cu) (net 2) (status 80000))
 (segment (start 40.005 29.845) (end 40.005 26.67) (width 0.254) (layer F.Cu) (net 2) (status 80000))
 (via (at 40.005 26.67) (size 0.889) (layers F.Cu B.Cu) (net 2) (status 80000))
 (segment (start 40.005 26.67) (end 40.005 24.765) (width 0.254) (layer B.Cu) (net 2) (status 80000))
 (segment (start 40.005 24.765) (end 34.29 19.05) (width 0.254) (layer B.Cu) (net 2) (status 80000))
 (segment (start 30.48 29.718) (end 30.48 26.67) (width 0.254) (layer F.Cu) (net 2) (status 80000))
 (segment (start 50.8 31.115) (end 48.895 29.21) (width 0.254) (layer B.Cu) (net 3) (status 80000))
 (segment (start 48.895 29.21) (end 38.735 29.21) (width 0.254) (layer B.Cu) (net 3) (status 80000))
 (via (at 38.735 29.21) (size 0.889) (layers F.Cu B.Cu) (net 3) (status 80000))
 (segment (start 38.735 29.21) (end 38.1 29.21) (width 0.254) (layer F.Cu) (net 3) (status 80000))
 (segment (start 38.1 29.21) (end 35.56 31.75) (width 0.254) (layer F.Cu) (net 3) (status 80000))
 (segment (start 35.56 31.75) (end 33.27 31.75) (width 0.254) (layer F.Cu) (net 3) (status 80000))
 (segment (start 44.45 24.38) (end 44.45 26.035) (width 0.254) (layer F.Cu) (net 4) (status 80000))
 (segment (start 44.45 26.035) (end 43.18 27.305) (width 0.254) (layer F.Cu) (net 4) (status 80000))
 (segment (start 43.18 27.305) (end 43.18 31.75) (width 0.254) (layer F.Cu) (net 4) (status 80000))
 (segment (start 43.18 31.75) (end 44.45 33.02) (width 0.254) (layer F.Cu) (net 4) (status 80000))
 (via (at 44.45 33.02) (size 0.889) (layers F.Cu B.Cu) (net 4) (status 80000))
 (segment (start 44.45 33.02) (end 45.085 33.655) (width 0.254) (layer B.Cu) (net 4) (status 80000))
 (segment (start 45.085 33.655) (end 50.8 33.655) (width 0.254) (layer B.Cu) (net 4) (status 80000))
 (segment (start 46.74 26.67) (end 50.8 26.67) (width 0.254) (layer F.Cu) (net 6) (status 80000))
 (segment (start 50.8 26.67) (end 51.435 27.305) (width 0.254) (layer F.Cu) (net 6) (status 80000))
 (segment (start 51.435 27.305) (end 52.07 27.305) (width 0.254) (layer F.Cu) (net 6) (status 80000))
 (segment (start 52.07 27.305) (end 52.07 37.465) (width 0.254) (layer F.Cu) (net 6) (status 80000))
 (segment (start 52.07 37.465) (end 50.8 38.735) (width 0.254) (layer F.Cu) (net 6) (status 80000))
 (segment (start 48.51 59.37) (end 48.26 59.055) (width 0.254) (layer F.Cu) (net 7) (status 80000))
 (segment (start 48.26 59.055) (end 35.56 71.755) (width 0.254) (layer F.Cu) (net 7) (status 80000))
 (segment (start 35.56 71.755) (end 35.56 81.915) (width 0.254) (layer F.Cu) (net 7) (status 80000))
 (segment (start 35.56 81.915) (end 35.31 82.23) (width 0.254) (layer F.Cu) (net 7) (status 80000))
 (segment (start 39.37 37.85) (end 39.37 39.37) (width 0.254) (layer F.Cu) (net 7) (status 80000))
 (segment (start 39.37 39.37) (end 40.64 40.64) (width 0.254) (layer F.Cu) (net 7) (status 80000))
 (via (at 40.64 40.64) (size 0.889) (layers F.Cu B.Cu) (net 7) (status 80000))
 (segment (start 40.64 40.64) (end 41.275 41.275) (width 0.254) (layer B.Cu) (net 7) (status 80000))
 (segment (start 41.275 41.275) (end 50.8 41.275) (width 0.254) (layer B.Cu) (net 7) (status 80000))
 (segment (start 50.8 41.275) (end 52.07 42.545) (width 0.254) (layer F.Cu) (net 7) (status 80000))
 (segment (start 52.07 42.545) (end 52.07 45.085) (width 0.254) (layer F.Cu) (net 7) (status 80000))
 (segment (start 52.07 45.085) (end 51.435 45.72) (width 0.254) (layer F.Cu) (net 7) (status 80000))
 (segment (start 51.435 45.72) (end 51.435 59.055) (width 0.254) (layer F.Cu) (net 7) (status 80000))
 (segment (start 51.435 59.055) (end 51.51 59.37) (width 0.254) (layer F.Cu) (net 7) (status 80000))
 (segment (start 37.58 31.545) (end 37.465 31.75) (width 0.254) (layer B.Cu) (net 7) (status 80000))
 (segment (start 37.465 31.75) (end 39.37 31.75) (width 0.254) (layer B.Cu) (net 7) (status 80000))
 (via (at 39.37 31.75) (size 0.889) (layers F.Cu B.Cu) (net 7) (status 80000))
 (segment (start 39.37 31.75) (end 39.37 37.85) (width 0.254) (layer F.Cu) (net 7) (status 80000))
 (segment (start 37.58 31.545) (end 37.465 31.75) (width 0.254) (layer B.Cu) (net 7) (status 80000))
 (segment (start 37.465 31.75) (end 37.465 30.48) (width 0.254) (layer B.Cu) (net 7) (status 80000))
 (segment (start 37.465 30.48) (end 36.195 29.21) (width 0.254) (layer B.Cu) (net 7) (status 80000))
 (via (at 36.195 29.21) (size 0.889) (layers F.Cu B.Cu) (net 7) (status 80000))
 (segment (start 36.195 29.21) (end 34.925 30.48) (width 0.254) (layer F.Cu) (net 7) (status 80000))
 (segment (start 34.925 30.48) (end 33.27 30.48) (width 0.254) (layer F.Cu) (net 7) (status 80000))
 (segment (start 51.51 59.37) (end 51.435 59.055) (width 0.254) (layer B.Cu) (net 7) (status 80000))
 (segment (start 51.435 59.055) (end 48.26 59.055) (width 0.254) (layer B.Cu) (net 7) (status 80000))
 (segment (start 48.26 59.055) (end 48.51 59.37) (width 0.254) (layer B.Cu) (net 7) (status 80000))
 (segment (start 36.08 31.545) (end 36.195 31.75) (width 0.254) (layer B.Cu) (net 1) (status 80000))
 (segment (start 36.195 31.75) (end 36.195 32.385) (width 0.254) (layer B.Cu) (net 1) (status 80000))
 (segment (start 36.195 32.385) (end 36.83 33.02) (width 0.254) (layer B.Cu) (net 1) (status 80000))
 (segment (start 36.83 33.02) (end 40.005 33.02) (width 0.254) (layer B.Cu) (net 1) (status 80000))
 (segment (start 40.005 33.02) (end 41.91 31.115) (width 0.254) (layer B.Cu) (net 1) (status 80000))
 (segment (start 41.91 31.115) (end 44.45 31.115) (width 0.254) (layer B.Cu) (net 1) (status 80000))
 (via (at 44.45 31.115) (size 0.889) (layers F.Cu B.Cu) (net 1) (status 80000))
 (segment (start 44.45 31.115) (end 45.085 30.48) (width 0.254) (layer F.Cu) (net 1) (status 80000))
 (segment (start 45.085 30.48) (end 46.74 30.48) (width 0.254) (layer F.Cu) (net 1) (status 80000))
 (segment (start 46.74 30.48) (end 48.895 30.48) (width 0.254) (layer F.Cu) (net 1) (status 80000))
 (segment (start 48.895 30.48) (end 50.8 28.575) (width 0.254) (layer F.Cu) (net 1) (status 80000))
 (segment (start 30.48 31.242) (end 30.48 31.115) (width 0.254) (layer F.Cu) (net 1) (status 80000))
 (segment (start 30.48 31.115) (end 31.115 30.48) (width 0.254) (layer F.Cu) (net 1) (status 80000))
 (segment (start 31.115 30.48) (end 31.75 30.48) (width 0.254) (layer F.Cu) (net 1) (status 80000))
 (segment (start 31.75 30.48) (end 31.75 22.225) (width 0.254) (layer F.Cu) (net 1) (status 80000))
 (via (at 31.75 22.225) (size 0.889) (layers F.Cu B.Cu) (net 1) (status 80000))
 (segment (start 31.75 22.225) (end 31.75 27.305) (width 0.254) (layer B.Cu) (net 1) (status 80000))
 (segment (start 31.75 27.305) (end 36.195 31.75) (width 0.254) (layer B.Cu) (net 1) (status 80000))
 (segment (start 36.195 31.75) (end 36.08 31.545) (width 0.254) (layer B.Cu) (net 1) (status 80000))
 (segment (start 30.48 34.29) (end 30.48 38.1) (width 0.254) (layer F.Cu) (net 1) (status 80000))
 (segment (start 30.48 34.29) (end 30.48 31.242) (width 0.254) (layer F.Cu) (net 1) (status 80000))
 (segment (start 30.48 38.1) (end 30.48 40.259) (width 0.254) (layer B.Cu) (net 1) (status 80000)))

